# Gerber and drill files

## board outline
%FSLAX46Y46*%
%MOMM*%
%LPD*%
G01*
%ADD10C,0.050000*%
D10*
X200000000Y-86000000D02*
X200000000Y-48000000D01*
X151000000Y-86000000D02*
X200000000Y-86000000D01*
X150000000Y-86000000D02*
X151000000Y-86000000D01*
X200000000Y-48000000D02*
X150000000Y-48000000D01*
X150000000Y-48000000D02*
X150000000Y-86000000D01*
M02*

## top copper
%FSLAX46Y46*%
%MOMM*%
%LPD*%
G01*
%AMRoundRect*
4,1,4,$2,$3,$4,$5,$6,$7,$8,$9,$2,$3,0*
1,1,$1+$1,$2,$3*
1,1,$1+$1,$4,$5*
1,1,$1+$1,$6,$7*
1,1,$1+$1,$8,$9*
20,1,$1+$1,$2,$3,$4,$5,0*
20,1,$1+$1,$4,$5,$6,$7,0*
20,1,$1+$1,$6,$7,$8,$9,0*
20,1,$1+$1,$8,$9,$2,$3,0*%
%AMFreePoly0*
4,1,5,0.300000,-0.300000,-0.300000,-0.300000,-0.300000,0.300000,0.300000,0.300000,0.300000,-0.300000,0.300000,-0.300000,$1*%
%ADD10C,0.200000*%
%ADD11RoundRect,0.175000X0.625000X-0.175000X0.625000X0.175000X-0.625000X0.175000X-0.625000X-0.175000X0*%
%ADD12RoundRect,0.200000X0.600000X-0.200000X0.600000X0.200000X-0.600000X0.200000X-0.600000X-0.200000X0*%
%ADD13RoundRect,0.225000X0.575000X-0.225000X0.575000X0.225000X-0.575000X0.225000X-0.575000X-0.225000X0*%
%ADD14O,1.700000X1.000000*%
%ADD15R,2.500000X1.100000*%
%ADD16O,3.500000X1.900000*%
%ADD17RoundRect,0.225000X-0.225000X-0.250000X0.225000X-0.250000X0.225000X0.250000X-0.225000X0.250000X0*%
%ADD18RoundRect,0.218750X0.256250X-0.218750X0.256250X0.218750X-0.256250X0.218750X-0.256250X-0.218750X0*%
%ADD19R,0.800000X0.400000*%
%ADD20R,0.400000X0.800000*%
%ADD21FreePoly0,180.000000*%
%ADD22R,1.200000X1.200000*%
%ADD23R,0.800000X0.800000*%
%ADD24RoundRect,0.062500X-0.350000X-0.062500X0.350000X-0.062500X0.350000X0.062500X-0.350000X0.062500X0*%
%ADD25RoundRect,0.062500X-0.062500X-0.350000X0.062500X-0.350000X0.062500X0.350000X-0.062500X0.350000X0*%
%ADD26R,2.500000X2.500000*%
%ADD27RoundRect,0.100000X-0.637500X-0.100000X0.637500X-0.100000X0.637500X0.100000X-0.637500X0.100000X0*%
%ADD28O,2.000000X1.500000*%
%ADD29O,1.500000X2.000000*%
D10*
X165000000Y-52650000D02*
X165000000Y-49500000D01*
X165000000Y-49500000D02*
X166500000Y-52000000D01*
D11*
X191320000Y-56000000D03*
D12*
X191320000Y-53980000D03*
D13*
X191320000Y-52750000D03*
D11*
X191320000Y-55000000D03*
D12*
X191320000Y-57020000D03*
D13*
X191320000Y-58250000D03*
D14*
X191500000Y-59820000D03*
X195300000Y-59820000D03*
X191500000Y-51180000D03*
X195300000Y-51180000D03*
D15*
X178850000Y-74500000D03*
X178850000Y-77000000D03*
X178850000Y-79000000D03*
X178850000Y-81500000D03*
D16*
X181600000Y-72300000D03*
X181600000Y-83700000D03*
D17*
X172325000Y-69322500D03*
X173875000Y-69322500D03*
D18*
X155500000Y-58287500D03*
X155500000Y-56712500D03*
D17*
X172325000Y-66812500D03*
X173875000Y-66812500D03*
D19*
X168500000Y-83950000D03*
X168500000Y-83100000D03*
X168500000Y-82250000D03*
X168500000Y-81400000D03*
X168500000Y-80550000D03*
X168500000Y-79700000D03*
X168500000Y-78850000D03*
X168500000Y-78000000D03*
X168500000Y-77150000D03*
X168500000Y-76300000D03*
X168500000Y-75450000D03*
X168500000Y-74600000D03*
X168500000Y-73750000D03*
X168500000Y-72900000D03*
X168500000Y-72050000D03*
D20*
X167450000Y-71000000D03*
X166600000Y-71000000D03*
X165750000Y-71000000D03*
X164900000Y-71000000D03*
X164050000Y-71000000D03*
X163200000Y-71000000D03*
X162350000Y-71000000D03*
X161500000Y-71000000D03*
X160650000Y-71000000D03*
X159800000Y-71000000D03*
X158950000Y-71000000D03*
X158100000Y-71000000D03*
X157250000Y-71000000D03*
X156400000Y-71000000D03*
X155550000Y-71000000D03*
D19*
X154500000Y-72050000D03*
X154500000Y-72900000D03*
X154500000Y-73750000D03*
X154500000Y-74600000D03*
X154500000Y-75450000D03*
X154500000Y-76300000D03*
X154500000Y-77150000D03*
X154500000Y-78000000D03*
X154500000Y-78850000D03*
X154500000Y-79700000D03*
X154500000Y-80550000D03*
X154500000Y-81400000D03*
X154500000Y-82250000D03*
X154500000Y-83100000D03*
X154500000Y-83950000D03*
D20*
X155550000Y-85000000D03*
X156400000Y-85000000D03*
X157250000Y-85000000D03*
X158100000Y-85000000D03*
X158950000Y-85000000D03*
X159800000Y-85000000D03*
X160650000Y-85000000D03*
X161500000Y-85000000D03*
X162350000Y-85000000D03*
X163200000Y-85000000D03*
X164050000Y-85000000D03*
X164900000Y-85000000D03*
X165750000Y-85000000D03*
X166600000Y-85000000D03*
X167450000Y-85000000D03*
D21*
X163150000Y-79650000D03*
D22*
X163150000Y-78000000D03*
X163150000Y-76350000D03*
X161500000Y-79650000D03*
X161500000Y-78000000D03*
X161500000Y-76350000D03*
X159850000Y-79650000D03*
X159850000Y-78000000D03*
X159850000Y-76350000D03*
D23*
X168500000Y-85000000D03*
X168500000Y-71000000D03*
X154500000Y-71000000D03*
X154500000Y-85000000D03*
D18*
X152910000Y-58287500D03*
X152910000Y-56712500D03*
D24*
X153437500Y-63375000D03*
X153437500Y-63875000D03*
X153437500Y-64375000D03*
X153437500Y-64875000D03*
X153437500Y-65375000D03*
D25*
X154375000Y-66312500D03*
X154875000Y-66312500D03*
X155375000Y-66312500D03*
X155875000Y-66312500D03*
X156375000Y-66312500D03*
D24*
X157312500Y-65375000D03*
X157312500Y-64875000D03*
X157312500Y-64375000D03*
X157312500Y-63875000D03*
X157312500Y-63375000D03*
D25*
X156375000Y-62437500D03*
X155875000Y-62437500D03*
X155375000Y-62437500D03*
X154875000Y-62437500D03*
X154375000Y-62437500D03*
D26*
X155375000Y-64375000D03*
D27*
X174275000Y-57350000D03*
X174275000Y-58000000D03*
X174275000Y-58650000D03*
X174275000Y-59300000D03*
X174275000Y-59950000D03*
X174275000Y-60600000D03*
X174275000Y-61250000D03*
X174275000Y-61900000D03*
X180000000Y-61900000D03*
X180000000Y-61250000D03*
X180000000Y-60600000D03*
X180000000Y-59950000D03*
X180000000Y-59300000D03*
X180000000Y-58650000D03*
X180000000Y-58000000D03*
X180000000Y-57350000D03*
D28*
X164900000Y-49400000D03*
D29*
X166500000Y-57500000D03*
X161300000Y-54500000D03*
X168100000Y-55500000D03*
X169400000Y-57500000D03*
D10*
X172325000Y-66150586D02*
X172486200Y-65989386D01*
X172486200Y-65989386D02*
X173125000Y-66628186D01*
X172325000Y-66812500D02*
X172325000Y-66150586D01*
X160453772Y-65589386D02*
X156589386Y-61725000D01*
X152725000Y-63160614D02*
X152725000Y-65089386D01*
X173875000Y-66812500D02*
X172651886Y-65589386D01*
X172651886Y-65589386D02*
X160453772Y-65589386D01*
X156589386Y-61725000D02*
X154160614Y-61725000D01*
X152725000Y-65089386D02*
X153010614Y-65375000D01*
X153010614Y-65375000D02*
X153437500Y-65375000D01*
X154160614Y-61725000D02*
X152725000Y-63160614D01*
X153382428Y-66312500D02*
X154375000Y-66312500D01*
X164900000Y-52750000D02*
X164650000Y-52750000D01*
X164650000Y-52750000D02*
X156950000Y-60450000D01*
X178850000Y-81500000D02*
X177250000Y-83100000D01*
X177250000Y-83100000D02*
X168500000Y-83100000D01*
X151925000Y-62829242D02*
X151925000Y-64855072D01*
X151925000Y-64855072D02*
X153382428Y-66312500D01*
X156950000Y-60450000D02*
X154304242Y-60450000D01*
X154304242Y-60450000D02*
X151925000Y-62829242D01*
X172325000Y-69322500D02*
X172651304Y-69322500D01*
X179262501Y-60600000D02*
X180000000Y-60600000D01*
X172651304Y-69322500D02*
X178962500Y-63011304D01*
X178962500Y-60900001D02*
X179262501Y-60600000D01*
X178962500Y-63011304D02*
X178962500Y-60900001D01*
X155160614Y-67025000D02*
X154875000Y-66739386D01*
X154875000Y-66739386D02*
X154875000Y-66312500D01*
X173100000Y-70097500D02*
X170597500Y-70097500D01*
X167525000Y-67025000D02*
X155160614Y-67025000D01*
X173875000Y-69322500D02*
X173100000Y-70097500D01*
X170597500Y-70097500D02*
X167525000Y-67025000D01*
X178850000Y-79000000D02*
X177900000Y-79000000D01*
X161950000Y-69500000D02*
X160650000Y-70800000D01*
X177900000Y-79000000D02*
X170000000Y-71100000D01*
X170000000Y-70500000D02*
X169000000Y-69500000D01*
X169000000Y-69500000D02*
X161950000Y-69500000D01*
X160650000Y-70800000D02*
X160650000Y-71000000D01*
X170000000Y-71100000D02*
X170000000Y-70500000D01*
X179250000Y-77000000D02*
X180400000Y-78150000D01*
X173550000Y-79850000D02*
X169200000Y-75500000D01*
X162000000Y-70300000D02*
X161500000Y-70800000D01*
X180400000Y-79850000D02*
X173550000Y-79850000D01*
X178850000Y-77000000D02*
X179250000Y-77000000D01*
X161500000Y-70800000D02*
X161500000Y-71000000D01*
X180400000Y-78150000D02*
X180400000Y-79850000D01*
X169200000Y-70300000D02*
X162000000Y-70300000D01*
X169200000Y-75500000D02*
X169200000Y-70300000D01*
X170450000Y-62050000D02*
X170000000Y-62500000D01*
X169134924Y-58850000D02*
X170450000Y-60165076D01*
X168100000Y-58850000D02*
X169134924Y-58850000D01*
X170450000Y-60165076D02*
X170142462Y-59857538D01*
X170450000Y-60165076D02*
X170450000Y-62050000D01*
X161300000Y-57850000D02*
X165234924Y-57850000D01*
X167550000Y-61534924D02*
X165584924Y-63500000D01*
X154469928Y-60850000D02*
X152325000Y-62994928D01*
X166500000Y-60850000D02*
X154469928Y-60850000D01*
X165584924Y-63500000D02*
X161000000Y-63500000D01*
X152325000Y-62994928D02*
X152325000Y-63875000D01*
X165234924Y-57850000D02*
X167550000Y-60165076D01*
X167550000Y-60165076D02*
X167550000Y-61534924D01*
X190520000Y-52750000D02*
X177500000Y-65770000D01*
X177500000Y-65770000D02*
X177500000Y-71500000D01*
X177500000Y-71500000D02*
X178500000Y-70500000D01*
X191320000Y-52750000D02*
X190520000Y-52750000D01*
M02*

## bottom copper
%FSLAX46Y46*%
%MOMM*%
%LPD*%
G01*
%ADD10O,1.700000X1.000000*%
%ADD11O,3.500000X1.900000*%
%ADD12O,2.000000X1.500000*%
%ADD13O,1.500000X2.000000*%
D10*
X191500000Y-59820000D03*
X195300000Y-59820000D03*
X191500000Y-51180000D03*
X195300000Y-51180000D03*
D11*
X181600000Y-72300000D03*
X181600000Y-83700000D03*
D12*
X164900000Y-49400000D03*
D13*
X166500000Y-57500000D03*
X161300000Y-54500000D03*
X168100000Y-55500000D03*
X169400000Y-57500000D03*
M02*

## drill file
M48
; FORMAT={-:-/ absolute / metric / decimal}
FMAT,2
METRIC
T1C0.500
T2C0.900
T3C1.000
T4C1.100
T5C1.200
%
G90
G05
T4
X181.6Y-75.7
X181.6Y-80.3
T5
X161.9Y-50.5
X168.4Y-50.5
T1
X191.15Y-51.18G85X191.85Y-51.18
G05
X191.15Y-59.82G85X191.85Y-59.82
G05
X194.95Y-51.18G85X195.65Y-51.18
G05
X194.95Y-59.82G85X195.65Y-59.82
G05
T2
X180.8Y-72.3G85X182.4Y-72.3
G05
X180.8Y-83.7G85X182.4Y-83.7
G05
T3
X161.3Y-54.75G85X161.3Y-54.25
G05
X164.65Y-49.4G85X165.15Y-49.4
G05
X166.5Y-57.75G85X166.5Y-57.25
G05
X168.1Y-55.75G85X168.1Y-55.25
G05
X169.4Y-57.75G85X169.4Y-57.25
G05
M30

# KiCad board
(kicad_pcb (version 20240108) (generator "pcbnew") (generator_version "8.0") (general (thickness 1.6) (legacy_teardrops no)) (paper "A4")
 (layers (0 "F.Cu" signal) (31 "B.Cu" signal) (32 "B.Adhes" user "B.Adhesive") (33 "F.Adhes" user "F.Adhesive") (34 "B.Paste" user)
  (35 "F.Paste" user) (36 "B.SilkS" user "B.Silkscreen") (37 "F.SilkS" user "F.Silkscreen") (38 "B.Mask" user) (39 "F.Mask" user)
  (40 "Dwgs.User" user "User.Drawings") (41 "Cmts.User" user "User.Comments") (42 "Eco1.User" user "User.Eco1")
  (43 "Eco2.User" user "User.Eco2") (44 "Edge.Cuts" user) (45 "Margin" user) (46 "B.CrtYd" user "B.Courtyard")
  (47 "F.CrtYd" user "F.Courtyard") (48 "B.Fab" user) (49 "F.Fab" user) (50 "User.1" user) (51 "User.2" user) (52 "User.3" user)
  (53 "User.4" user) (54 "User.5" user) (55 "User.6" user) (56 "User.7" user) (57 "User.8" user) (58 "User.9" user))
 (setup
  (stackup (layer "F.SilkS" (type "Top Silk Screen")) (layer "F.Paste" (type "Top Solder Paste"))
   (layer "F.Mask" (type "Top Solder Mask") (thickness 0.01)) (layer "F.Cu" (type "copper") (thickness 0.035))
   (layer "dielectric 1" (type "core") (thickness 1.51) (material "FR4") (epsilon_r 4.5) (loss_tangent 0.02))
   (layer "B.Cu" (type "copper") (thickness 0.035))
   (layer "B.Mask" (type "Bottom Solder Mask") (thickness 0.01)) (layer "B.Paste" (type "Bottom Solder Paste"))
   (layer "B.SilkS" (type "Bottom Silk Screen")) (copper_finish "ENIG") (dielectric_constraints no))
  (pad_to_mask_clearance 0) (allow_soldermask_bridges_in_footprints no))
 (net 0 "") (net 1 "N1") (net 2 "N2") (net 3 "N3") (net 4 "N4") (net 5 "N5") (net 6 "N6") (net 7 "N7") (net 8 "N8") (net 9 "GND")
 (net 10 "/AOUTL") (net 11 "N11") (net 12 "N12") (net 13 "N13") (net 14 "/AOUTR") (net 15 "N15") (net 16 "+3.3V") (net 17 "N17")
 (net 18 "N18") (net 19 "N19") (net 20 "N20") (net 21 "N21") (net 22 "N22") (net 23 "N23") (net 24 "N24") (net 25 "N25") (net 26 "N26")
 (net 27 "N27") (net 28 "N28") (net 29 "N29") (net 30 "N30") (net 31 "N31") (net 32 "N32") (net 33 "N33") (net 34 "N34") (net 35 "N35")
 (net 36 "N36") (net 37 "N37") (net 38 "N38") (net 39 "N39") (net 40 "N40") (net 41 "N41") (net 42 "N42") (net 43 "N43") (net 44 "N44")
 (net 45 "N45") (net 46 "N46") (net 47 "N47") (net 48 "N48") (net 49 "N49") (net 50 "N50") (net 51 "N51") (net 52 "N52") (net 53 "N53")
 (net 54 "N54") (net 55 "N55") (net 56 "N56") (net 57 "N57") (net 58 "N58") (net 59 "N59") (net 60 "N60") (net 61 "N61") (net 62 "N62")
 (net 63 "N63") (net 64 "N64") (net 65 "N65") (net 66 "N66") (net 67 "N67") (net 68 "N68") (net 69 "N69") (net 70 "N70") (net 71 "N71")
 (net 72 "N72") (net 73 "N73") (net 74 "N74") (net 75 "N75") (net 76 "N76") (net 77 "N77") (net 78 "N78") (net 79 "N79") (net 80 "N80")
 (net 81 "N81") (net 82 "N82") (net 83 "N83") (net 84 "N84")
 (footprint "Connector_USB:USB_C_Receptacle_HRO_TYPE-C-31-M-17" (layer "F.Cu") (at 194.5 55.5 90)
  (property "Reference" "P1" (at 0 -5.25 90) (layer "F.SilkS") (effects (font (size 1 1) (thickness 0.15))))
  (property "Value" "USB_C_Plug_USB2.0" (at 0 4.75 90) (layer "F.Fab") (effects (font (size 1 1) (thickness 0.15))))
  (pad "A5" smd roundrect (at -0.5 -3.18 90) (size 0.7 1.6) (layers "F.Cu" "F.Paste" "F.Mask") (roundrect_rratio 0.25) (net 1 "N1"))
  (pad "A9" smd roundrect (at 1.52 -3.18 90) (size 0.8 1.6) (layers "F.Cu" "F.Paste" "F.Mask") (roundrect_rratio 0.25) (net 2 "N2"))
  (pad "A12" smd roundrect (at 2.75 -3.18 90) (size 0.9 1.6) (layers "F.Cu" "F.Paste" "F.Mask") (roundrect_rratio 0.25) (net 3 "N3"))
  (pad "B5" smd roundrect (at 0.5 -3.18 90) (size 0.7 1.6) (layers "F.Cu" "F.Paste" "F.Mask") (roundrect_rratio 0.25) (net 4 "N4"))
  (pad "B9" smd roundrect (at -1.52 -3.18 90) (size 0.8 1.6) (layers "F.Cu" "F.Paste" "F.Mask") (roundrect_rratio 0.25) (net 2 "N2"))
  (pad "B12" smd roundrect (at -2.75 -3.18 90) (size 0.9 1.6) (layers "F.Cu" "F.Paste" "F.Mask") (roundrect_rratio 0.25) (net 3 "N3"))
  (pad "S1" thru_hole oval (at -4.32 -3 90) (size 1 1.7) (drill oval 0.5 1.2) (layers "*.Cu" "*.Mask") (remove_unused_layers no)
   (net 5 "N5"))
  (pad "S1" thru_hole oval (at -4.32 0.8 90) (size 1 1.7) (drill oval 0.5 1.2) (layers "*.Cu" "*.Mask") (remove_unused_layers no)
   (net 5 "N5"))
  (pad "S1" thru_hole oval (at 4.32 -3 90) (size 1 1.7) (drill oval 0.5 1.2) (layers "*.Cu" "*.Mask") (remove_unused_layers no) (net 5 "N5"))
  (pad "S1" thru_hole oval (at 4.32 0.8 90) (size 1 1.7) (drill oval 0.5 1.2) (layers "*.Cu" "*.Mask") (remove_unused_layers no)
   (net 5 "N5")))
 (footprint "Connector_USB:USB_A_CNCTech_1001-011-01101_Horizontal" (layer "F.Cu") (at 188.5 78)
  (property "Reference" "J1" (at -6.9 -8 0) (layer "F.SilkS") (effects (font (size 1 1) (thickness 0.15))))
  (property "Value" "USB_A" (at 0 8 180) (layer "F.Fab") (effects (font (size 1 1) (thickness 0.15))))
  (pad "" np_thru_hole circle (at -6.9 -2.3) (size 1.1 1.1) (drill 1.1) (layers "*.Cu" "*.Mask"))
  (pad "" np_thru_hole circle (at -6.9 2.3) (size 1.1 1.1) (drill 1.1) (layers "*.Cu" "*.Mask"))
  (pad "1" smd rect (at -9.65 -3.5) (size 2.5 1.1) (layers "F.Cu" "F.Paste" "F.Mask") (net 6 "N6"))
  (pad "2" smd rect (at -9.65 -1) (size 2.5 1.1) (layers "F.Cu" "F.Paste" "F.Mask") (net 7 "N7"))
  (pad "3" smd rect (at -9.65 1) (size 2.5 1.1) (layers "F.Cu" "F.Paste" "F.Mask") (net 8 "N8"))
  (pad "4" smd rect (at -9.65 3.5) (size 2.5 1.1) (layers "F.Cu" "F.Paste" "F.Mask") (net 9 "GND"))
  (pad "5" thru_hole oval (at -6.9 -5.7) (size 3.5 1.9) (drill oval 2.5 0.9) (layers "*.Cu" "*.Mask") (remove_unused_layers no)
   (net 9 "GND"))
  (pad "5" thru_hole oval (at -6.9 5.7) (size 3.5 1.9) (drill oval 2.5 0.9) (layers "*.Cu" "*.Mask") (remove_unused_layers no) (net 9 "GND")))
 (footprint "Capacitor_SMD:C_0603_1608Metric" (layer "F.Cu") (at 173.1 69.3225)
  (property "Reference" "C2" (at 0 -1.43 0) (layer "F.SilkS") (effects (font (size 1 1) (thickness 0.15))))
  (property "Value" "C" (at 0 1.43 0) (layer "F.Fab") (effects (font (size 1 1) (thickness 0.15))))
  (pad "1" smd roundrect (at -0.775 0) (size 0.9 0.95) (layers "F.Cu" "F.Paste" "F.Mask") (roundrect_rratio 0.25) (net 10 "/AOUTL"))
  (pad "2" smd roundrect (at 0.775 0) (size 0.9 0.95) (layers "F.Cu" "F.Paste" "F.Mask") (roundrect_rratio 0.25) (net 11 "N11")))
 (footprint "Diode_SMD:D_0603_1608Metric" (layer "F.Cu") (at 155.5 57.5 90)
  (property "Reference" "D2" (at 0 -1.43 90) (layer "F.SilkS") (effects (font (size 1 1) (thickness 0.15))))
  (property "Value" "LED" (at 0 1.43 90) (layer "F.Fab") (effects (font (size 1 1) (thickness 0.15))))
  (pad "1" smd roundrect (at -0.7875 0 90) (size 0.875 0.95) (layers "F.Cu" "F.Paste" "F.Mask") (roundrect_rratio 0.25) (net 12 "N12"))
  (pad "2" smd roundrect (at 0.7875 0 90) (size 0.875 0.95) (layers "F.Cu" "F.Paste" "F.Mask") (roundrect_rratio 0.25) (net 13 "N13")))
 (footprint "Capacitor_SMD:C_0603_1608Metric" (layer "F.Cu") (at 173.1 66.8125)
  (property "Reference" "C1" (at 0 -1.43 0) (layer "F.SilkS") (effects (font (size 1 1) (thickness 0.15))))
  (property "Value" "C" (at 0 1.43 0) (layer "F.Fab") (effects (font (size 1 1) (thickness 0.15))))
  (pad "1" smd roundrect (at -0.775 0) (size 0.9 0.95) (layers "F.Cu" "F.Paste" "F.Mask") (roundrect_rratio 0.25) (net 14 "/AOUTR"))
  (pad "2" smd roundrect (at 0.775 0) (size 0.9 0.95) (layers "F.Cu" "F.Paste" "F.Mask") (roundrect_rratio 0.25) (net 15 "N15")))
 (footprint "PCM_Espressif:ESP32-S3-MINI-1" (layer "F.Cu") (at 161.5 78 180)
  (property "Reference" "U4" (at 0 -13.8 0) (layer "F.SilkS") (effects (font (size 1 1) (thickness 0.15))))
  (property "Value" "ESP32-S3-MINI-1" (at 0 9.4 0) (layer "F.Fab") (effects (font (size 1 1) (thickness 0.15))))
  (pad "1" smd rect (at -7 -5.95 270) (size 0.4 0.8) (layers "F.Cu" "F.Paste" "F.Mask") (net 9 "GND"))
  (pad "2" smd rect (at -7 -5.1 270) (size 0.4 0.8) (layers "F.Cu" "F.Paste" "F.Mask") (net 9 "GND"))
  (pad "3" smd rect (at -7 -4.25 270) (size 0.4 0.8) (layers "F.Cu" "F.Paste" "F.Mask") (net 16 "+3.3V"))
  (pad "4" smd rect (at -7 -3.4 270) (size 0.4 0.8) (layers "F.Cu" "F.Paste" "F.Mask") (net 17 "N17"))
  (pad "5" smd rect (at -7 -2.55 270) (size 0.4 0.8) (layers "F.Cu" "F.Paste" "F.Mask") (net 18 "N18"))
  (pad "6" smd rect (at -7 -1.7 270) (size 0.4 0.8) (layers "F.Cu" "F.Paste" "F.Mask") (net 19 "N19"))
  (pad "7" smd rect (at -7 -0.85 270) (size 0.4 0.8) (layers "F.Cu" "F.Paste" "F.Mask") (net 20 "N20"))
  (pad "8" smd rect (at -7 0 270) (size 0.4 0.8) (layers "F.Cu" "F.Paste" "F.Mask") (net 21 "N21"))
  (pad "9" smd rect (at -7 0.85 270) (size 0.4 0.8) (layers "F.Cu" "F.Paste" "F.Mask") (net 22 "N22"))
  (pad "10" smd rect (at -7 1.7 270) (size 0.4 0.8) (layers "F.Cu" "F.Paste" "F.Mask") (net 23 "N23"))
  (pad "11" smd rect (at -7 2.55 270) (size 0.4 0.8) (layers "F.Cu" "F.Paste" "F.Mask") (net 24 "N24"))
  (pad "12" smd rect (at -7 3.4 270) (size 0.4 0.8) (layers "F.Cu" "F.Paste" "F.Mask") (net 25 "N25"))
  (pad "13" smd rect (at -7 4.25 270) (size 0.4 0.8) (layers "F.Cu" "F.Paste" "F.Mask") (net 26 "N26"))
  (pad "14" smd rect (at -7 5.1 270) (size 0.4 0.8) (layers "F.Cu" "F.Paste" "F.Mask") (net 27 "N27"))
  (pad "15" smd rect (at -7 5.95 270) (size 0.4 0.8) (layers "F.Cu" "F.Paste" "F.Mask") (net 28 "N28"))
  (pad "16" smd rect (at -5.95 7 180) (size 0.4 0.8) (layers "F.Cu" "F.Paste" "F.Mask") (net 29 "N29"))
  (pad "17" smd rect (at -5.1 7 180) (size 0.4 0.8) (layers "F.Cu" "F.Paste" "F.Mask") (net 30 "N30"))
  (pad "18" smd rect (at -4.25 7 180) (size 0.4 0.8) (layers "F.Cu" "F.Paste" "F.Mask") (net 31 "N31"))
  (pad "19" smd rect (at -3.4 7 180) (size 0.4 0.8) (layers "F.Cu" "F.Paste" "F.Mask") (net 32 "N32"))
  (pad "20" smd rect (at -2.55 7 180) (size 0.4 0.8) (layers "F.Cu" "F.Paste" "F.Mask") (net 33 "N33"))
  (pad "21" smd rect (at -1.7 7 180) (size 0.4 0.8) (layers "F.Cu" "F.Paste" "F.Mask") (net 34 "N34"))
  (pad "22" smd rect (at -0.85 7 180) (size 0.4 0.8) (layers "F.Cu" "F.Paste" "F.Mask") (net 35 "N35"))
  (pad "23" smd rect (at 0 7 180) (size 0.4 0.8) (layers "F.Cu" "F.Paste" "F.Mask") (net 7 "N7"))
  (pad "24" smd rect (at 0.85 7 180) (size 0.4 0.8) (layers "F.Cu" "F.Paste" "F.Mask") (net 8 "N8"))
  (pad "25" smd rect (at 1.7 7 180) (size 0.4 0.8) (layers "F.Cu" "F.Paste" "F.Mask") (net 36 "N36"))
  (pad "26" smd rect (at 2.55 7 180) (size 0.4 0.8) (layers "F.Cu" "F.Paste" "F.Mask") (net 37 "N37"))
  (pad "27" smd rect (at 3.4 7 180) (size 0.4 0.8) (layers "F.Cu" "F.Paste" "F.Mask") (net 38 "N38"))
  (pad "28" smd rect (at 4.25 7 180) (size 0.4 0.8) (layers "F.Cu" "F.Paste" "F.Mask") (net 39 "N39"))
  (pad "29" smd rect (at 5.1 7 180) (size 0.4 0.8) (layers "F.Cu" "F.Paste" "F.Mask") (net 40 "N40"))
  (pad "30" smd rect (at 5.95 7 180) (size 0.4 0.8) (layers "F.Cu" "F.Paste" "F.Mask") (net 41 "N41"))
  (pad "31" smd rect (at 7 5.95 270) (size 0.4 0.8) (layers "F.Cu" "F.Paste" "F.Mask") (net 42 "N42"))
  (pad "32" smd rect (at 7 5.1 270) (size 0.4 0.8) (layers "F.Cu" "F.Paste" "F.Mask") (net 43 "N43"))
  (pad "33" smd rect (at 7 4.25 270) (size 0.4 0.8) (layers "F.Cu" "F.Paste" "F.Mask") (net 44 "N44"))
  (pad "34" smd rect (at 7 3.4 270) (size 0.4 0.8) (layers "F.Cu" "F.Paste" "F.Mask") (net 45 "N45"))
  (pad "35" smd rect (at 7 2.55 270) (size 0.4 0.8) (layers "F.Cu" "F.Paste" "F.Mask") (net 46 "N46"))
  (pad "36" smd rect (at 7 1.7 270) (size 0.4 0.8) (layers "F.Cu" "F.Paste" "F.Mask") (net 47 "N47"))
  (pad "37" smd rect (at 7 0.85 270) (size 0.4 0.8) (layers "F.Cu" "F.Paste" "F.Mask") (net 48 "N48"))
  (pad "38" smd rect (at 7 0 270) (size 0.4 0.8) (layers "F.Cu" "F.Paste" "F.Mask") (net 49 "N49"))
  (pad "39" smd rect (at 7 -0.85 270) (size 0.4 0.8) (layers "F.Cu" "F.Paste" "F.Mask") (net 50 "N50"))
  (pad "40" smd rect (at 7 -1.7 270) (size 0.4 0.8) (layers "F.Cu" "F.Paste" "F.Mask") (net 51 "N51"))
  (pad "41" smd rect (at 7 -2.55 270) (size 0.4 0.8) (layers "F.Cu" "F.Paste" "F.Mask") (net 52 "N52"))
  (pad "42" smd rect (at 7 -3.4 270) (size 0.4 0.8) (layers "F.Cu" "F.Paste" "F.Mask") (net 9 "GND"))
  (pad "43" smd rect (at 7 -4.25 270) (size 0.4 0.8) (layers "F.Cu" "F.Paste" "F.Mask") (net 9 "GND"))
  (pad "44" smd rect (at 7 -5.1 270) (size 0.4 0.8) (layers "F.Cu" "F.Paste" "F.Mask") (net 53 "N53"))
  (pad "45" smd rect (at 7 -5.95 270) (size 0.4 0.8) (layers "F.Cu" "F.Paste" "F.Mask") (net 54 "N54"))
  (pad "46" smd rect (at 5.95 -7 180) (size 0.4 0.8) (layers "F.Cu" "F.Paste" "F.Mask") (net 9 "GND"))
  (pad "47" smd rect (at 5.1 -7 180) (size 0.4 0.8) (layers "F.Cu" "F.Paste" "F.Mask") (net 9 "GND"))
  (pad "48" smd rect (at 4.25 -7 180) (size 0.4 0.8) (layers "F.Cu" "F.Paste" "F.Mask") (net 9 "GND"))
  (pad "49" smd rect (at 3.4 -7 180) (size 0.4 0.8) (layers "F.Cu" "F.Paste" "F.Mask") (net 9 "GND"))
  (pad "50" smd rect (at 2.55 -7 180) (size 0.4 0.8) (layers "F.Cu" "F.Paste" "F.Mask") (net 9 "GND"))
  (pad "51" smd rect (at 1.7 -7 180) (size 0.4 0.8) (layers "F.Cu" "F.Paste" "F.Mask") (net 9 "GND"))
  (pad "52" smd rect (at 0.85 -7 180) (size 0.4 0.8) (layers "F.Cu" "F.Paste" "F.Mask") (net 9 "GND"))
  (pad "53" smd rect (at 0 -7 180) (size 0.4 0.8) (layers "F.Cu" "F.Paste" "F.Mask") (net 9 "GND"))
  (pad "54" smd rect (at -0.85 -7 180) (size 0.4 0.8) (layers "F.Cu" "F.Paste" "F.Mask") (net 9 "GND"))
  (pad "55" smd rect (at -1.7 -7 180) (size 0.4 0.8) (layers "F.Cu" "F.Paste" "F.Mask") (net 9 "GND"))
  (pad "56" smd rect (at -2.55 -7 180) (size 0.4 0.8) (layers "F.Cu" "F.Paste" "F.Mask") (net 9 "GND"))
  (pad "57" smd rect (at -3.4 -7 180) (size 0.4 0.8) (layers "F.Cu" "F.Paste" "F.Mask") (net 9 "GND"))
  (pad "58" smd rect (at -4.25 -7 180) (size 0.4 0.8) (layers "F.Cu" "F.Paste" "F.Mask") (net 9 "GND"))
  (pad "59" smd rect (at -5.1 -7 180) (size 0.4 0.8) (layers "F.Cu" "F.Paste" "F.Mask") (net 9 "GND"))
  (pad "60" smd rect (at -5.95 -7 180) (size 0.4 0.8) (layers "F.Cu" "F.Paste" "F.Mask") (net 9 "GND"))
  (pad "61" smd custom (at -1.65 -1.65 180) (size 0.6 0.6) (layers "F.Cu" "F.Paste" "F.Mask") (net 9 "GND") (zone_connect 2)
   (thermal_bridge_angle 45) (options (clearance outline) (anchor rect)) (primitives))
  (pad "61" smd rect (at -1.65 0 180) (size 1.2 1.2) (layers "F.Cu" "F.Paste" "F.Mask") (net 9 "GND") (zone_connect 2))
  (pad "61" smd rect (at -1.65 1.65 180) (size 1.2 1.2) (layers "F.Cu" "F.Paste" "F.Mask") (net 9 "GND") (zone_connect 2))
  (pad "61" smd rect (at 0 -1.65 180) (size 1.2 1.2) (layers "F.Cu" "F.Paste" "F.Mask") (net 9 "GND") (zone_connect 2))
  (pad "61" smd rect (at 0 0 180) (size 1.2 1.2) (layers "F.Cu" "F.Paste" "F.Mask") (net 9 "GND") (zone_connect 2))
  (pad "61" smd rect (at 0 1.65 180) (size 1.2 1.2) (layers "F.Cu" "F.Paste" "F.Mask") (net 9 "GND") (zone_connect 2))
  (pad "61" smd rect (at 1.65 -1.65 180) (size 1.2 1.2) (layers "F.Cu" "F.Paste" "F.Mask") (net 9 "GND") (zone_connect 2))
  (pad "61" smd rect (at 1.65 0 180) (size 1.2 1.2) (layers "F.Cu" "F.Paste" "F.Mask") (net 9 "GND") (zone_connect 2))
  (pad "61" smd rect (at 1.65 1.65 180) (size 1.2 1.2) (layers "F.Cu" "F.Paste" "F.Mask") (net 9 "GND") (zone_connect 2))
  (pad "62" smd rect (at -7 -7) (size 0.8 0.8) (layers "F.Cu" "F.Paste" "F.Mask") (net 9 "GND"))
  (pad "63" smd rect (at -7 7) (size 0.8 0.8) (layers "F.Cu" "F.Paste" "F.Mask") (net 9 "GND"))
  (pad "64" smd rect (at 7 7) (size 0.8 0.8) (layers "F.Cu" "F.Paste" "F.Mask") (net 9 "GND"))
  (pad "65" smd rect (at 7 -7) (size 0.8 0.8) (layers "F.Cu" "F.Paste" "F.Mask") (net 9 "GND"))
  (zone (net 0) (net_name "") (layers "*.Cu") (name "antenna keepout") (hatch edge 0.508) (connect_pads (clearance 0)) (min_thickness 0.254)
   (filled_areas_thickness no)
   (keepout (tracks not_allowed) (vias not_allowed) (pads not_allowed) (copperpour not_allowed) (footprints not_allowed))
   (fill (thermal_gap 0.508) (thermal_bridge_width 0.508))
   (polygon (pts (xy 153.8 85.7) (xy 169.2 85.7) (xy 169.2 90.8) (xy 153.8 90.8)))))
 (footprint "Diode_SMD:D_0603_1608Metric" (layer "F.Cu") (at 152.91 57.5 90)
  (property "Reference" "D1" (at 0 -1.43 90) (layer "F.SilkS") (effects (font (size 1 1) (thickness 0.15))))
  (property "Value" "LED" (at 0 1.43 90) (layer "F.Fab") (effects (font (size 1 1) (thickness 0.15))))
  (pad "1" smd roundrect (at -0.7875 0 90) (size 0.875 0.95) (layers "F.Cu" "F.Paste" "F.Mask") (roundrect_rratio 0.25) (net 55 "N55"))
  (pad "2" smd roundrect (at 0.7875 0 90) (size 0.875 0.95) (layers "F.Cu" "F.Paste" "F.Mask") (roundrect_rratio 0.25) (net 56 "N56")))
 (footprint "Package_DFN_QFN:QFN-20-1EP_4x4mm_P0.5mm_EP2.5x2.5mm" (layer "F.Cu") (at 155.375 64.375)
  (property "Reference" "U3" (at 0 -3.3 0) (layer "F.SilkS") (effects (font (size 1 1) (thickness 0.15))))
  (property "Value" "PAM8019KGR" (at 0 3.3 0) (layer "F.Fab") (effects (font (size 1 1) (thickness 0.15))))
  (pad "" smd roundrect (at -0.625 -0.625) (size 1.01 1.01) (layers "F.Paste") (roundrect_rratio 0.247525))
  (pad "" smd roundrect (at -0.625 0.625) (size 1.01 1.01) (layers "F.Paste") (roundrect_rratio 0.247525))
  (pad "" smd roundrect (at 0.625 -0.625) (size 1.01 1.01) (layers "F.Paste") (roundrect_rratio 0.247525))
  (pad "" smd roundrect (at 0.625 0.625) (size 1.01 1.01) (layers "F.Paste") (roundrect_rratio 0.247525))
  (pad "1" smd roundrect (at -1.9375 -1) (size 0.825 0.25) (layers "F.Cu" "F.Paste" "F.Mask") (roundrect_rratio 0.25) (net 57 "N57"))
  (pad "2" smd roundrect (at -1.9375 -0.5) (size 0.825 0.25) (layers "F.Cu" "F.Paste" "F.Mask") (roundrect_rratio 0.25) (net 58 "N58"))
  (pad "3" smd roundrect (at -1.9375 0) (size 0.825 0.25) (layers "F.Cu" "F.Paste" "F.Mask") (roundrect_rratio 0.25) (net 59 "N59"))
  (pad "4" smd roundrect (at -1.9375 0.5) (size 0.825 0.25) (layers "F.Cu" "F.Paste" "F.Mask") (roundrect_rratio 0.25) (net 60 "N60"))
  (pad "5" smd roundrect (at -1.9375 1) (size 0.825 0.25) (layers "F.Cu" "F.Paste" "F.Mask") (roundrect_rratio 0.25) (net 15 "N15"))
  (pad "6" smd roundrect (at -1 1.9375) (size 0.25 0.825) (layers "F.Cu" "F.Paste" "F.Mask") (roundrect_rratio 0.25) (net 9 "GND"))
  (pad "7" smd roundrect (at -0.5 1.9375) (size 0.25 0.825) (layers "F.Cu" "F.Paste" "F.Mask") (roundrect_rratio 0.25) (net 11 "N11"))
  (pad "8" smd roundrect (at 0 1.9375) (size 0.25 0.825) (layers "F.Cu" "F.Paste" "F.Mask") (roundrect_rratio 0.25) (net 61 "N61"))
  (pad "9" smd roundrect (at 0.5 1.9375) (size 0.25 0.825) (layers "F.Cu" "F.Paste" "F.Mask") (roundrect_rratio 0.25) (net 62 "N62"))
  (pad "10" smd roundrect (at 1 1.9375) (size 0.25 0.825) (layers "F.Cu" "F.Paste" "F.Mask") (roundrect_rratio 0.25) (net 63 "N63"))
  (pad "11" smd roundrect (at 1.9375 1) (size 0.825 0.25) (layers "F.Cu" "F.Paste" "F.Mask") (roundrect_rratio 0.25) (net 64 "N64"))
  (pad "12" smd roundrect (at 1.9375 0.5) (size 0.825 0.25) (layers "F.Cu" "F.Paste" "F.Mask") (roundrect_rratio 0.25) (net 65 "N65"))
  (pad "13" smd roundrect (at 1.9375 0) (size 0.825 0.25) (layers "F.Cu" "F.Paste" "F.Mask") (roundrect_rratio 0.25) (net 16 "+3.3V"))
  (pad "14" smd roundrect (at 1.9375 -0.5) (size 0.825 0.25) (layers "F.Cu" "F.Paste" "F.Mask") (roundrect_rratio 0.25) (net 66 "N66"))
  (pad "15" smd roundrect (at 1.9375 -1) (size 0.825 0.25) (layers "F.Cu" "F.Paste" "F.Mask") (roundrect_rratio 0.25) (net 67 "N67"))
  (pad "16" smd roundrect (at 1 -1.9375) (size 0.25 0.825) (layers "F.Cu" "F.Paste" "F.Mask") (roundrect_rratio 0.25) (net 16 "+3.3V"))
  (pad "17" smd roundrect (at 0.5 -1.9375) (size 0.25 0.825) (layers "F.Cu" "F.Paste" "F.Mask") (roundrect_rratio 0.25) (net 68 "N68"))
  (pad "18" smd roundrect (at 0 -1.9375) (size 0.25 0.825) (layers "F.Cu" "F.Paste" "F.Mask") (roundrect_rratio 0.25) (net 9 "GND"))
  (pad "19" smd roundrect (at -0.5 -1.9375) (size 0.25 0.825) (layers "F.Cu" "F.Paste" "F.Mask") (roundrect_rratio 0.25) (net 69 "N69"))
  (pad "20" smd roundrect (at -1 -1.9375) (size 0.25 0.825) (layers "F.Cu" "F.Paste" "F.Mask") (roundrect_rratio 0.25) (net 16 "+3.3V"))
  (pad "21" smd rect (at 0 0) (size 2.5 2.5) (layers "F.Cu" "F.Mask") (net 9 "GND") (zone_connect 2)))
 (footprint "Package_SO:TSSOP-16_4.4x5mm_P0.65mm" (layer "F.Cu") (at 177.1375 59.625)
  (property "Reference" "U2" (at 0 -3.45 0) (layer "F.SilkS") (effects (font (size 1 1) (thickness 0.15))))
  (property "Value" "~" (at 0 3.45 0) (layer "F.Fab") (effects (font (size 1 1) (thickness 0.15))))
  (pad "1" smd roundrect (at -2.8625 -2.275) (size 1.475 0.4) (layers "F.Cu" "F.Paste" "F.Mask") (roundrect_rratio 0.25) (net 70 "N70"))
  (pad "2" smd roundrect (at -2.8625 -1.625) (size 1.475 0.4) (layers "F.Cu" "F.Paste" "F.Mask") (roundrect_rratio 0.25) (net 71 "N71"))
  (pad "3" smd roundrect (at -2.8625 -0.975) (size 1.475 0.4) (layers "F.Cu" "F.Paste" "F.Mask") (roundrect_rratio 0.25) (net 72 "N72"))
  (pad "4" smd roundrect (at -2.8625 -0.325) (size 1.475 0.4) (layers "F.Cu" "F.Paste" "F.Mask") (roundrect_rratio 0.25) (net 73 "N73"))
  (pad "5" smd roundrect (at -2.8625 0.325) (size 1.475 0.4) (layers "F.Cu" "F.Paste" "F.Mask") (roundrect_rratio 0.25) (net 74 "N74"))
  (pad "6" smd roundrect (at -2.8625 0.975) (size 1.475 0.4) (layers "F.Cu" "F.Paste" "F.Mask") (roundrect_rratio 0.25) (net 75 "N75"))
  (pad "7" smd roundrect (at -2.8625 1.625) (size 1.475 0.4) (layers "F.Cu" "F.Paste" "F.Mask") (roundrect_rratio 0.25) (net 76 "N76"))
  (pad "8" smd roundrect (at -2.8625 2.275) (size 1.475 0.4) (layers "F.Cu" "F.Paste" "F.Mask") (roundrect_rratio 0.25) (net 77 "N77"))
  (pad "9" smd roundrect (at 2.8625 2.275) (size 1.475 0.4) (layers "F.Cu" "F.Paste" "F.Mask") (roundrect_rratio 0.25) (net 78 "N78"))
  (pad "10" smd roundrect (at 2.8625 1.625) (size 1.475 0.4) (layers "F.Cu" "F.Paste" "F.Mask") (roundrect_rratio 0.25) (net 14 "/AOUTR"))
  (pad "11" smd roundrect (at 2.8625 0.975) (size 1.475 0.4) (layers "F.Cu" "F.Paste" "F.Mask") (roundrect_rratio 0.25) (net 10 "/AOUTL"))
  (pad "12" smd roundrect (at 2.8625 0.325) (size 1.475 0.4) (layers "F.Cu" "F.Paste" "F.Mask") (roundrect_rratio 0.25) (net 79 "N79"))
  (pad "13" smd roundrect (at 2.8625 -0.325) (size 1.475 0.4) (layers "F.Cu" "F.Paste" "F.Mask") (roundrect_rratio 0.25) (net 9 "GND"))
  (pad "14" smd roundrect (at 2.8625 -0.975) (size 1.475 0.4) (layers "F.Cu" "F.Paste" "F.Mask") (roundrect_rratio 0.25) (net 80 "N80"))
  (pad "15" smd roundrect (at 2.8625 -1.625) (size 1.475 0.4) (layers "F.Cu" "F.Paste" "F.Mask") (roundrect_rratio 0.25) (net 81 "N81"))
  (pad "16" smd roundrect (at 2.8625 -2.275) (size 1.475 0.4) (layers "F.Cu" "F.Paste" "F.Mask") (roundrect_rratio 0.25) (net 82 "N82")))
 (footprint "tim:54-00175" (layer "F.Cu") (at 164.9 47 -90)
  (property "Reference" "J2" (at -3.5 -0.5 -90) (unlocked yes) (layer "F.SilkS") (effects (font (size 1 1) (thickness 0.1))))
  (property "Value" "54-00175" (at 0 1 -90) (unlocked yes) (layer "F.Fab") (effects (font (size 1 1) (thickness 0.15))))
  (pad "" np_thru_hole circle (at 3.5 -3.5 90) (size 1.2 1.2) (drill 1.2) (layers "F&B.Cu" "*.Mask"))
  (pad "" np_thru_hole circle (at 3.5 3 90) (size 1.2 1.2) (drill 1.2) (layers "F&B.Cu" "*.Mask"))
  (pad "1" thru_hole oval (at 2.4 0) (size 2 1.5) (drill oval 1.5 1) (layers "*.Cu" "*.Mask") (remove_unused_layers no) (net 9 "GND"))
  (pad "2" thru_hole oval (at 10.5 -1.6 90) (size 2 1.5) (drill oval 1.5 1) (layers "*.Cu" "*.Mask") (remove_unused_layers no)
   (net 58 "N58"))
  (pad "3" thru_hole oval (at 7.5 3.6 90) (size 2 1.5) (drill oval 1.5 1) (layers "*.Cu" "*.Mask") (remove_unused_layers no) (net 66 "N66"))
  (pad "4" thru_hole oval (at 8.5 -3.2 90) (size 2 1.5) (drill oval 1.5 1) (layers "*.Cu" "*.Mask") (remove_unused_layers no) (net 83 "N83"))
  (pad "5" thru_hole oval (at 10.5 -4.5 90) (size 2 1.5) (drill oval 1.5 1) (layers "*.Cu" "*.Mask") (remove_unused_layers no)
   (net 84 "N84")))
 (gr_line (start 165 52.65) (end 165 49.5) (stroke (width 0.2) (type default)) (layer "F.Cu") (net 9))
 (gr_line (start 165 49.5) (end 166.5 52) (stroke (width 0.2) (type default)) (layer "F.Cu") (net 9))
 (gr_line (start 200 86) (end 200 48) (stroke (width 0.05) (type default)) (layer "Edge.Cuts"))
 (gr_line (start 151 86) (end 200 86) (stroke (width 0.05) (type default)) (layer "Edge.Cuts"))
 (gr_line (start 150 86) (end 151 86) (stroke (width 0.05) (type default)) (layer "Edge.Cuts"))
 (gr_line (start 200 48) (end 150 48) (stroke (width 0.05) (type default)) (layer "Edge.Cuts"))
 (gr_line (start 150 48) (end 150 86) (stroke (width 0.05) (type default)) (layer "Edge.Cuts"))
 (segment (start 172.325 66.150586) (end 172.4862 65.989386) (width 0.2) (layer "F.Cu") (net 14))
 (segment (start 172.4862 65.989386) (end 173.125 66.628186) (width 0.2) (layer "F.Cu") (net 14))
 (segment (start 172.325 66.8125) (end 172.325 66.150586) (width 0.2) (layer "F.Cu") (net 14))
 (segment (start 160.453772 65.589386) (end 156.589386 61.725) (width 0.2) (layer "F.Cu") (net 15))
 (segment (start 152.725 63.160614) (end 152.725 65.089386) (width 0.2) (layer "F.Cu") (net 15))
 (segment (start 173.875 66.8125) (end 172.651886 65.589386) (width 0.2) (layer "F.Cu") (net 15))
 (segment (start 172.651886 65.589386) (end 160.453772 65.589386) (width 0.2) (layer "F.Cu") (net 15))
 (segment (start 156.589386 61.725) (end 154.160614 61.725) (width 0.2) (layer "F.Cu") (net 15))
 (segment (start 152.725 65.089386) (end 153.010614 65.375) (width 0.2) (layer "F.Cu") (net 15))
 (segment (start 153.010614 65.375) (end 153.4375 65.375) (width 0.2) (layer "F.Cu") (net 15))
 (segment (start 154.160614 61.725) (end 152.725 63.160614) (width 0.2) (layer "F.Cu") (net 15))
 (segment (start 153.382428 66.3125) (end 154.375 66.3125) (width 0.2) (layer "F.Cu") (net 9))
 (segment (start 164.9 52.75) (end 164.65 52.75) (width 0.2) (layer "F.Cu") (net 9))
 (segment (start 164.65 52.75) (end 156.95 60.45) (width 0.2) (layer "F.Cu") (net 9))
 (segment (start 178.85 81.5) (end 177.25 83.1) (width 0.2) (layer "F.Cu") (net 9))
 (segment (start 177.25 83.1) (end 168.5 83.1) (width 0.2) (layer "F.Cu") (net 9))
 (segment (start 151.925 62.829242) (end 151.925 64.855072) (width 0.2) (layer "F.Cu") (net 9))
 (segment (start 151.925 64.855072) (end 153.382428 66.3125) (width 0.2) (layer "F.Cu") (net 9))
 (segment (start 156.95 60.45) (end 154.304242 60.45) (width 0.2) (layer "F.Cu") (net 9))
 (segment (start 154.304242 60.45) (end 151.925 62.829242) (width 0.2) (layer "F.Cu") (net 9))
 (segment (start 172.325 69.3225) (end 172.651304 69.3225) (width 0.2) (layer "F.Cu") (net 10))
 (segment (start 179.262501 60.6) (end 180 60.6) (width 0.2) (layer "F.Cu") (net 10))
 (segment (start 172.651304 69.3225) (end 178.9625 63.011304) (width 0.2) (layer "F.Cu") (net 10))
 (segment (start 178.9625 60.900001) (end 179.262501 60.6) (width 0.2) (layer "F.Cu") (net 10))
 (segment (start 178.9625 63.011304) (end 178.9625 60.900001) (width 0.2) (layer "F.Cu") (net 10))
 (segment (start 155.160614 67.025) (end 154.875 66.739386) (width 0.2) (layer "F.Cu") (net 11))
 (segment (start 154.875 66.739386) (end 154.875 66.3125) (width 0.2) (layer "F.Cu") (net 11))
 (segment (start 173.1 70.0975) (end 170.5975 70.0975) (width 0.2) (layer "F.Cu") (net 11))
 (segment (start 167.525 67.025) (end 155.160614 67.025) (width 0.2) (layer "F.Cu") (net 11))
 (segment (start 173.875 69.3225) (end 173.1 70.0975) (width 0.2) (layer "F.Cu") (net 11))
 (segment (start 170.5975 70.0975) (end 167.525 67.025) (width 0.2) (layer "F.Cu") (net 11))
 (segment (start 178.85 79) (end 177.9 79) (width 0.2) (layer "F.Cu") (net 8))
 (segment (start 161.95 69.5) (end 160.65 70.8) (width 0.2) (layer "F.Cu") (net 8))
 (segment (start 177.9 79) (end 170 71.1) (width 0.2) (layer "F.Cu") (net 8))
 (segment (start 170 70.5) (end 169 69.5) (width 0.2) (layer "F.Cu") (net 8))
 (segment (start 169 69.5) (end 161.95 69.5) (width 0.2) (layer "F.Cu") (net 8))
 (segment (start 160.65 70.8) (end 160.65 71) (width 0.2) (layer "F.Cu") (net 8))
 (segment (start 170 71.1) (end 170 70.5) (width 0.2) (layer "F.Cu") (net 8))
 (segment (start 179.25 77) (end 180.4 78.15) (width 0.2) (layer "F.Cu") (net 7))
 (segment (start 173.55 79.85) (end 169.2 75.5) (width 0.2) (layer "F.Cu") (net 7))
 (segment (start 162 70.3) (end 161.5 70.8) (width 0.2) (layer "F.Cu") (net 7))
 (segment (start 180.4 79.85) (end 173.55 79.85) (width 0.2) (layer "F.Cu") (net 7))
 (segment (start 178.85 77) (end 179.25 77) (width 0.2) (layer "F.Cu") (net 7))
 (segment (start 161.5 70.8) (end 161.5 71) (width 0.2) (layer "F.Cu") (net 7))
 (segment (start 180.4 78.15) (end 180.4 79.85) (width 0.2) (layer "F.Cu") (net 7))
 (segment (start 169.2 70.3) (end 162 70.3) (width 0.2) (layer "F.Cu") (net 7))
 (segment (start 169.2 75.5) (end 169.2 70.3) (width 0.2) (layer "F.Cu") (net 7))
 (segment (start 170.45 62.05) (end 170 62.5) (width 0.2) (layer "F.Cu") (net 84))
 (segment (start 169.134924 58.85) (end 170.45 60.165076) (width 0.2) (layer "F.Cu") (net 84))
 (segment (start 168.1 58.85) (end 169.134924 58.85) (width 0.2) (layer "F.Cu") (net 84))
 (segment (start 170.45 60.165076) (end 170.142462 59.857538) (width 0.2) (layer "F.Cu") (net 84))
 (segment (start 170.45 60.165076) (end 170.45 62.05) (width 0.2) (layer "F.Cu") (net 84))
 (segment (start 161.3 57.85) (end 165.234924 57.85) (width 0.2) (layer "F.Cu") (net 58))
 (segment (start 167.55 61.534924) (end 165.584924 63.5) (width 0.2) (layer "F.Cu") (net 58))
 (segment (start 154.469928 60.85) (end 152.325 62.994928) (width 0.2) (layer "F.Cu") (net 58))
 (segment (start 166.5 60.85) (end 154.469928 60.85) (width 0.2) (layer "F.Cu") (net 58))
 (segment (start 165.584924 63.5) (end 161 63.5) (width 0.2) (layer "F.Cu") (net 58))
 (segment (start 152.325 62.994928) (end 152.325 63.875) (width 0.2) (layer "F.Cu") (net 58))
 (segment (start 165.234924 57.85) (end 167.55 60.165076) (width 0.2) (layer "F.Cu") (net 58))
 (segment (start 167.55 60.165076) (end 167.55 61.534924) (width 0.2) (layer "F.Cu") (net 58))
 (segment (start 190.52 52.75) (end 177.5 65.77) (width 0.2) (layer "F.Cu") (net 3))
 (segment (start 177.5 65.77) (end 177.5 71.5) (width 0.2) (layer "F.Cu") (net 3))
 (segment (start 177.5 71.5) (end 178.5 70.5) (width 0.2) (layer "F.Cu") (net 3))
 (segment (start 191.32 52.75) (end 190.52 52.75) (width 0.2) (layer "F.Cu") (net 3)))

